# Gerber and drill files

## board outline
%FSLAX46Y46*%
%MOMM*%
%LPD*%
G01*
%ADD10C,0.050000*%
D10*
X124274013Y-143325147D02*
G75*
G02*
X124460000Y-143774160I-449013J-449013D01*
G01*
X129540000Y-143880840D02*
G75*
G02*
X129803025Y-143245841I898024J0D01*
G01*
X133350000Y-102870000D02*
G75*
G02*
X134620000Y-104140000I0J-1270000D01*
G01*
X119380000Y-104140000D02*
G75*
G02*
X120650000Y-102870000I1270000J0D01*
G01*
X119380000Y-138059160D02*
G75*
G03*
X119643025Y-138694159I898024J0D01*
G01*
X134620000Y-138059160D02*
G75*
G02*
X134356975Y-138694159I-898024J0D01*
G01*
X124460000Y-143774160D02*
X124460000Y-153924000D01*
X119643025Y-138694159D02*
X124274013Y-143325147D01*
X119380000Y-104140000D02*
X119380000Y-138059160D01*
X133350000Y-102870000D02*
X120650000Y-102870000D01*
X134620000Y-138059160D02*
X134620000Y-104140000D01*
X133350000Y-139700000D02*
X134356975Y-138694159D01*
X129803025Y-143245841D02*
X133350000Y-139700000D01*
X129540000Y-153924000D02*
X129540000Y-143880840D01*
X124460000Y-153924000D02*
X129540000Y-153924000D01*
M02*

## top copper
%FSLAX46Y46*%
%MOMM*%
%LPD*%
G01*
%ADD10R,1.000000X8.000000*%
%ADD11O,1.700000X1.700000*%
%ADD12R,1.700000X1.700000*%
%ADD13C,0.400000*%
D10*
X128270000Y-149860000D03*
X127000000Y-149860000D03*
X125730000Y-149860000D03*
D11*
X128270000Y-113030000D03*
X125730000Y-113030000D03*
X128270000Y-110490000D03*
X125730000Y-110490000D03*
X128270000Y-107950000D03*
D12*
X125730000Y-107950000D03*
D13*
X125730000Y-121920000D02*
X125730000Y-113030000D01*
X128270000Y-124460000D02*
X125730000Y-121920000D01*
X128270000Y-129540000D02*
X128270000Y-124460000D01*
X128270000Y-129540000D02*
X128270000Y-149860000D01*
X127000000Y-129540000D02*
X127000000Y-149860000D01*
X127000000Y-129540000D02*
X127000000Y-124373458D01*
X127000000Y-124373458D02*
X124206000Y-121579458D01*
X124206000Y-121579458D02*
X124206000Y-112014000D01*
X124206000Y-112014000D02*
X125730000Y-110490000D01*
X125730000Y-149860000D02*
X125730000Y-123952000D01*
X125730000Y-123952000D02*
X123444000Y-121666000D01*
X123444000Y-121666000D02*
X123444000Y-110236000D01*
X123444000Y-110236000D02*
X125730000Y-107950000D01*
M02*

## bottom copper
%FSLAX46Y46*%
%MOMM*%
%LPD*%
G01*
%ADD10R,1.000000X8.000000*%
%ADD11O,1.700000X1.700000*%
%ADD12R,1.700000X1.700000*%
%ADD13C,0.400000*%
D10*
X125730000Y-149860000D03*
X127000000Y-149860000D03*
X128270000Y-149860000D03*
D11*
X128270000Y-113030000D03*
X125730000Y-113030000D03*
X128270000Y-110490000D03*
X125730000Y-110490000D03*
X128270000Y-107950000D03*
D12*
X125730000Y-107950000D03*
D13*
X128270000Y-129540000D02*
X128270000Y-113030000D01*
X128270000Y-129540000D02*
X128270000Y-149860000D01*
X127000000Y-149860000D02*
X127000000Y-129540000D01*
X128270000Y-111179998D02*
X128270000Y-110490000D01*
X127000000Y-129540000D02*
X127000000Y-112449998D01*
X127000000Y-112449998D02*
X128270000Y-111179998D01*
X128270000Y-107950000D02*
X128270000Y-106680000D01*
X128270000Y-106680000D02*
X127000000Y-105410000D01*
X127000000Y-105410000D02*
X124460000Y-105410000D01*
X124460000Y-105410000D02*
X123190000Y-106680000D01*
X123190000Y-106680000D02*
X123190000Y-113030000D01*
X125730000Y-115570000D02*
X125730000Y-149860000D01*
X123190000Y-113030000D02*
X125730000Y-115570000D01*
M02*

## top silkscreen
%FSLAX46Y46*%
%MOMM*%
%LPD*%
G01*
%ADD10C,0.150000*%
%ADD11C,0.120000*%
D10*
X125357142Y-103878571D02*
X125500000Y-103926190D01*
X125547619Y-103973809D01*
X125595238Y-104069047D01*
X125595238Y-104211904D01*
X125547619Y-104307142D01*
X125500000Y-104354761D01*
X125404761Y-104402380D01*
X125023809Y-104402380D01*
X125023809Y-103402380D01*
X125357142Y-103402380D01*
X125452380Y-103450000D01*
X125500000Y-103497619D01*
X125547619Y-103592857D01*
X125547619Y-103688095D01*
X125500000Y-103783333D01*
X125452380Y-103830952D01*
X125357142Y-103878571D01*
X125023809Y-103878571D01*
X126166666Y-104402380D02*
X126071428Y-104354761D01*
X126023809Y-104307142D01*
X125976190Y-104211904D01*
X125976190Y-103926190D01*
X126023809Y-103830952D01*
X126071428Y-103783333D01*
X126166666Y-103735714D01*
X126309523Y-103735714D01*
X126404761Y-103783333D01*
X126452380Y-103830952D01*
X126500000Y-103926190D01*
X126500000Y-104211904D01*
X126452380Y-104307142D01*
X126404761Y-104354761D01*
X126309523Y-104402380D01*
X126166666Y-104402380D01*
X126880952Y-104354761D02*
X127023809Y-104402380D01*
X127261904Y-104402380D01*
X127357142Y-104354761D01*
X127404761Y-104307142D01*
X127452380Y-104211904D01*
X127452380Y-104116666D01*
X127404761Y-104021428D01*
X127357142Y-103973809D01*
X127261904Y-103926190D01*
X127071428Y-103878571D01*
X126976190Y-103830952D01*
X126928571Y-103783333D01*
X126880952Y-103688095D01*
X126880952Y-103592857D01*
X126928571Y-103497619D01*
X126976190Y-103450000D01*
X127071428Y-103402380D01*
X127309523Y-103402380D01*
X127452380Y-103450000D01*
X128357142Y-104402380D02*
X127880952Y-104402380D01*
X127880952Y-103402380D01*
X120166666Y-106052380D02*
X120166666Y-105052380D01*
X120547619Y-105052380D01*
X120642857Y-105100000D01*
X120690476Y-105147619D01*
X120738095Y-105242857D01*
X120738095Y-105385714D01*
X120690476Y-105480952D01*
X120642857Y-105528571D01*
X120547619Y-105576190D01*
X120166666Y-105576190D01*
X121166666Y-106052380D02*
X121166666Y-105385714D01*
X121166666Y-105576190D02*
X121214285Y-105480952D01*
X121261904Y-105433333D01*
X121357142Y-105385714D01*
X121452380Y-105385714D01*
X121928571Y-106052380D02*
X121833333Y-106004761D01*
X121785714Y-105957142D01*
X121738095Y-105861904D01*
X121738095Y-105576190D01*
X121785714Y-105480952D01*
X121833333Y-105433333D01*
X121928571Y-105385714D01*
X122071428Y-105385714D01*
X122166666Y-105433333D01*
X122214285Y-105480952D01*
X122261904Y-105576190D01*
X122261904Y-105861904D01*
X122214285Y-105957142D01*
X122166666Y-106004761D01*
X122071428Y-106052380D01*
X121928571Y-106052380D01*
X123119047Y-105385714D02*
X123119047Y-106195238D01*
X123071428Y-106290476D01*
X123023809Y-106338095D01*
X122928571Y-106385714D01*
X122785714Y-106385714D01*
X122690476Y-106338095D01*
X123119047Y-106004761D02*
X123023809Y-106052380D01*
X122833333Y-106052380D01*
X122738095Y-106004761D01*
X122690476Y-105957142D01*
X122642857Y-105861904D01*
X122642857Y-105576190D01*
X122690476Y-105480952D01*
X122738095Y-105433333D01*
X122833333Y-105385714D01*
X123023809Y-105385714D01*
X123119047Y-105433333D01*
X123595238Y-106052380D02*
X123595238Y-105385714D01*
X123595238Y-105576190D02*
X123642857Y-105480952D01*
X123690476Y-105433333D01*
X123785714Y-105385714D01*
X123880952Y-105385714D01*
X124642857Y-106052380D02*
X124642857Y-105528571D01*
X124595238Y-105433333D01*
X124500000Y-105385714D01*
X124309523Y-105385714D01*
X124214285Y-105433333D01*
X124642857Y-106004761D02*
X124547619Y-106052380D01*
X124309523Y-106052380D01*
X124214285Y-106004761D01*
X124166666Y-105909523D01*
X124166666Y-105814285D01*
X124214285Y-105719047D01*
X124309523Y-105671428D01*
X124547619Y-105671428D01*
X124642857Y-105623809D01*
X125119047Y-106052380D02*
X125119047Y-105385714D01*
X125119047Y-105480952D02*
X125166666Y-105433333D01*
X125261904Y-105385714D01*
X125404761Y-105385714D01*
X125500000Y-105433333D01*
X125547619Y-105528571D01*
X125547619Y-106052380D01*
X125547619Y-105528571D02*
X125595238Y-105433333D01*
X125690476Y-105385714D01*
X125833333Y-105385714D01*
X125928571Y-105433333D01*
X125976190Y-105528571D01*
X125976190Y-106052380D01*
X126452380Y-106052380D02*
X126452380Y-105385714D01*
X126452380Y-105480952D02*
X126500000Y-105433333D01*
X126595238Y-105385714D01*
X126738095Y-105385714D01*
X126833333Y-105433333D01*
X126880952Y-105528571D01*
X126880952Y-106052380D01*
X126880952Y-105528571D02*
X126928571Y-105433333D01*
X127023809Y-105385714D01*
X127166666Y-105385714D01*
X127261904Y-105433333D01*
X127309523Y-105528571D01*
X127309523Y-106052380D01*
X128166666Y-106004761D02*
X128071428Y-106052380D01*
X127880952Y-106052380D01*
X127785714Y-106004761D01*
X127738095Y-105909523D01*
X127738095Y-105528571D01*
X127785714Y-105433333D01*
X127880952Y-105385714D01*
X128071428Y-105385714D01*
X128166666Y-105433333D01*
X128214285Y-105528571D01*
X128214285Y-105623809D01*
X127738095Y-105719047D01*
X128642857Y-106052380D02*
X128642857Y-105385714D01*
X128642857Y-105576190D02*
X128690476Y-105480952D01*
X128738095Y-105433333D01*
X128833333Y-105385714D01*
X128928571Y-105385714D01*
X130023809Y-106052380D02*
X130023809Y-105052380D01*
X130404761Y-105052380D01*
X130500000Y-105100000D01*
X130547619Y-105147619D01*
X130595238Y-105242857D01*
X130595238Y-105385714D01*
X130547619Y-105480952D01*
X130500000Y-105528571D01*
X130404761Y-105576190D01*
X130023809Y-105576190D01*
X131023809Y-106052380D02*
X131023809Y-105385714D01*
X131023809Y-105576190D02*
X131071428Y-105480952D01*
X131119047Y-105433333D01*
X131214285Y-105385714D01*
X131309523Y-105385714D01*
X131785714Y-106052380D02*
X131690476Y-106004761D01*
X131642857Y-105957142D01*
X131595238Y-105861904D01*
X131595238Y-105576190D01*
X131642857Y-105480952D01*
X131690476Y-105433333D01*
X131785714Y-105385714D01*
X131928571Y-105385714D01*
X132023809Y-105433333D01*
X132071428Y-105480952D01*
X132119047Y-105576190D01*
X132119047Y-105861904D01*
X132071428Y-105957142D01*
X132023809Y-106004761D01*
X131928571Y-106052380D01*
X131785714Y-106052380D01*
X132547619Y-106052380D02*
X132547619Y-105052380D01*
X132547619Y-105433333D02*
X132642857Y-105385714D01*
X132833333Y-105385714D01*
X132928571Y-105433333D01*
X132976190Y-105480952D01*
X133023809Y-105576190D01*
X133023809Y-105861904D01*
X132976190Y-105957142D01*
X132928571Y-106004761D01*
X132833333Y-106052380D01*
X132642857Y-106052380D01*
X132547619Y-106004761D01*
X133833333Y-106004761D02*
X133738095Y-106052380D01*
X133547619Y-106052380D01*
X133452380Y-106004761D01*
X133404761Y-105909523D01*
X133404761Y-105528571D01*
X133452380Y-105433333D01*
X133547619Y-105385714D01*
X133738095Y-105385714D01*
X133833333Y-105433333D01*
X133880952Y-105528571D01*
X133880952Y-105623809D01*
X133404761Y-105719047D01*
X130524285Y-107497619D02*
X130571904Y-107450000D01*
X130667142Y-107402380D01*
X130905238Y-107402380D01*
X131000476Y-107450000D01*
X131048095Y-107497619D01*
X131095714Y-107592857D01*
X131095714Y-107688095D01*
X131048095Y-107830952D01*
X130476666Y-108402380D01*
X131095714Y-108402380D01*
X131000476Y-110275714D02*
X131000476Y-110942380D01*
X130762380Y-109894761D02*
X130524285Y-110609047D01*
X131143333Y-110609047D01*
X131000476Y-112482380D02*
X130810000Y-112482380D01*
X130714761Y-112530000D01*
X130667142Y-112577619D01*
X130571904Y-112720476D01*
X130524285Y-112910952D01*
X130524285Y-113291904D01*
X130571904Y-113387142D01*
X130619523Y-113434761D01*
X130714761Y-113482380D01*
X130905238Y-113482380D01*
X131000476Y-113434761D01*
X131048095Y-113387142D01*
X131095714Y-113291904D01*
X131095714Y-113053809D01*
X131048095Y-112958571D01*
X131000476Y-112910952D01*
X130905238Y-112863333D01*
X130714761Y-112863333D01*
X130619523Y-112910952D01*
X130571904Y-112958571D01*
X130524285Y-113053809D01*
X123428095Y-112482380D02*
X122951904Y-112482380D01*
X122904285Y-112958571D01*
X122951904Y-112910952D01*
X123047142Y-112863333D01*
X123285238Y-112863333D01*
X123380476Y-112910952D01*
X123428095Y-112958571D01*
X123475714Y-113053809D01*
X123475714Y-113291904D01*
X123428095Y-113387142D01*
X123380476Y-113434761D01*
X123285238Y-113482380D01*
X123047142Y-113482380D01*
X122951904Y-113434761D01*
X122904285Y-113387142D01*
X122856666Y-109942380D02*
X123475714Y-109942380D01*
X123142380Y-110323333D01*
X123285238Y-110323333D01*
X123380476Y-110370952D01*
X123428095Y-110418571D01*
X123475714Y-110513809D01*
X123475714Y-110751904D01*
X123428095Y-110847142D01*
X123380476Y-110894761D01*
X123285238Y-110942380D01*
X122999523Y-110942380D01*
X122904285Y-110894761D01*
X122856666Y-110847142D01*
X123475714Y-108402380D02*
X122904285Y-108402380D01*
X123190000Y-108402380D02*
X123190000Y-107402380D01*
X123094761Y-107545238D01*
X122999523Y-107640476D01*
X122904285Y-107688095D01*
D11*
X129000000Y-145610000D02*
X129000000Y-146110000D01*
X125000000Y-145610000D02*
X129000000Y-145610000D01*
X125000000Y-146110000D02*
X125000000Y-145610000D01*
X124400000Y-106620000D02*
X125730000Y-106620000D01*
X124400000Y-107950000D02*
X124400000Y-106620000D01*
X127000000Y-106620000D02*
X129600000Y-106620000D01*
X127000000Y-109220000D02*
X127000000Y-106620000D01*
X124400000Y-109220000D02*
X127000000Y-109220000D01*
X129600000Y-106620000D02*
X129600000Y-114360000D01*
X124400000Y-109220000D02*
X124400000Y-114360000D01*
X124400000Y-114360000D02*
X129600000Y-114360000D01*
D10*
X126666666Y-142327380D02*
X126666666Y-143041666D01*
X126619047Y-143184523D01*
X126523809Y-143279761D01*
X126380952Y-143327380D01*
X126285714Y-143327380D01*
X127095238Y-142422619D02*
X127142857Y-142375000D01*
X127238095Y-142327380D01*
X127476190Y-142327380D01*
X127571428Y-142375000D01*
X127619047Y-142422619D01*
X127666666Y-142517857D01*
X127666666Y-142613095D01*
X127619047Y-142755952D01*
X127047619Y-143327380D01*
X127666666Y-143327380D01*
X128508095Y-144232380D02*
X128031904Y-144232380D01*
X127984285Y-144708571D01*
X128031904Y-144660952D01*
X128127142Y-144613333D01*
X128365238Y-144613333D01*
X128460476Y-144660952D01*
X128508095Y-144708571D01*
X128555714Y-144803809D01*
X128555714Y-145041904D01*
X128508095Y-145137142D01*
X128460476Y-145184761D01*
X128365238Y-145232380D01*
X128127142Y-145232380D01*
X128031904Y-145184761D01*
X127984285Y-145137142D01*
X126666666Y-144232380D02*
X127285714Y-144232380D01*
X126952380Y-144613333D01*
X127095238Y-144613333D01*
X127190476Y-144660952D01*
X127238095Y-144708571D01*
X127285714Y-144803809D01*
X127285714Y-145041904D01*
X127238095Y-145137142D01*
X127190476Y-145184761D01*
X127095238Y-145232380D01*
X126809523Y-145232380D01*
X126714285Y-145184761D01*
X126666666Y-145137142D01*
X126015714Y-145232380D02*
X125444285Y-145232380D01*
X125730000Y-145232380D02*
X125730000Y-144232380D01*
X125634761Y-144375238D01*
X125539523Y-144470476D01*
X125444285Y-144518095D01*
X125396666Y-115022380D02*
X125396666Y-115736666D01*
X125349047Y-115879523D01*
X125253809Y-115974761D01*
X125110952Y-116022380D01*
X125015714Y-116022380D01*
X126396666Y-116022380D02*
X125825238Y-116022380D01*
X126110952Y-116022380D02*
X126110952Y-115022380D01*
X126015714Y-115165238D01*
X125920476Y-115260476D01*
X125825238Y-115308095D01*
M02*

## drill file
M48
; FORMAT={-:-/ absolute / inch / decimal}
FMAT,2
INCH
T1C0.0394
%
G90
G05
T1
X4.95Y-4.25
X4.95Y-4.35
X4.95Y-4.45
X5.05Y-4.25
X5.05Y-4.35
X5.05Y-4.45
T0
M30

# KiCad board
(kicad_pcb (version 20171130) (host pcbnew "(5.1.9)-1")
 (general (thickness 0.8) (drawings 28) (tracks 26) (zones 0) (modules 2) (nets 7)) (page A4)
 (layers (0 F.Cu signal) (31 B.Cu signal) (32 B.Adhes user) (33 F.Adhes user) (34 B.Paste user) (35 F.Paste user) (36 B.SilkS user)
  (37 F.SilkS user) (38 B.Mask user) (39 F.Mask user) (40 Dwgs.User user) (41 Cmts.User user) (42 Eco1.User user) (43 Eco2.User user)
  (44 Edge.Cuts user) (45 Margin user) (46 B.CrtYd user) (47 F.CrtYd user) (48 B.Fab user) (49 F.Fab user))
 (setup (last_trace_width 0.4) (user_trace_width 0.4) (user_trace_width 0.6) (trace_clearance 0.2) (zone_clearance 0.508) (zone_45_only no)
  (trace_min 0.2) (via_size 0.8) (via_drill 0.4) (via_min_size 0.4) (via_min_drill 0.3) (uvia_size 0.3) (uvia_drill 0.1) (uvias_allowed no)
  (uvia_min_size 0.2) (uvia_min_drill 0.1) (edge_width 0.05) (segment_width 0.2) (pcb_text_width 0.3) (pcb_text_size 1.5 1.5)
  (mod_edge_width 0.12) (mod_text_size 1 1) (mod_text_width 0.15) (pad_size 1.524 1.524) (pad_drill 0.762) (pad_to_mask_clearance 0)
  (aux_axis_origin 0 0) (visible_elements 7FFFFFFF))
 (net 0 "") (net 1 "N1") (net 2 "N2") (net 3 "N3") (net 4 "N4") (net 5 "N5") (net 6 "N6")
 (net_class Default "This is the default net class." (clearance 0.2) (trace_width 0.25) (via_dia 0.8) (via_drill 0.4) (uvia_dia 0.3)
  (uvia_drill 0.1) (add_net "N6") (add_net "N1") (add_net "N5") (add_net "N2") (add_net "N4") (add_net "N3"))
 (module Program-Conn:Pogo (layer F.Cu) (at 127 149.86)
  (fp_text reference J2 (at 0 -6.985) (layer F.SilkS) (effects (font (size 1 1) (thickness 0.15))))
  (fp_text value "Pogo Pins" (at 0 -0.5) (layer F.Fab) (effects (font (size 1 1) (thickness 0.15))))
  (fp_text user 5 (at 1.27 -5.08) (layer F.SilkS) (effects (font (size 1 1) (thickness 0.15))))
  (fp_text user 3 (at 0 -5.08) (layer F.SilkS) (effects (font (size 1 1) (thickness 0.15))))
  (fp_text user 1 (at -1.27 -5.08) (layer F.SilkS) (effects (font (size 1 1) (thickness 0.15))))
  (fp_line (start 2 -4.25) (end 2 -3.75) (layer F.SilkS) (width 0.12))
  (fp_line (start -2 -4.25) (end 2 -4.25) (layer F.SilkS) (width 0.12))
  (fp_line (start -2 -3.75) (end -2 -4.25) (layer F.SilkS) (width 0.12))
  (pad 2 smd rect (at -1.27 0) (size 1 8) (layers B.Cu B.Paste B.Mask) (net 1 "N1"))
  (pad 4 smd rect (at 0 0) (size 1 8) (layers B.Cu B.Paste B.Mask) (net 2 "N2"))
  (pad 6 smd rect (at 1.27 0) (size 1 8) (layers B.Cu B.Paste B.Mask) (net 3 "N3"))
  (pad 5 smd rect (at 1.27 0) (size 1 8) (layers F.Cu F.Paste F.Mask) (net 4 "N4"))
  (pad 3 smd rect (at 0 0) (size 1 8) (layers F.Cu F.Paste F.Mask) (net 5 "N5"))
  (pad 1 smd rect (at -1.27 0) (size 1 8) (layers F.Cu F.Paste F.Mask) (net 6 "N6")))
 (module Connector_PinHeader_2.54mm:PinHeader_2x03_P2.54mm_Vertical (layer F.Cu) (at 125.73 107.95)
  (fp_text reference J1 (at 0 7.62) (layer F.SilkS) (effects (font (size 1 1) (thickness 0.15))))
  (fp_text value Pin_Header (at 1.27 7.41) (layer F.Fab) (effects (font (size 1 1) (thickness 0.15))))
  (fp_line (start -1.33 -1.33) (end 0 -1.33) (layer F.SilkS) (width 0.12))
  (fp_line (start -1.33 0) (end -1.33 -1.33) (layer F.SilkS) (width 0.12))
  (fp_line (start 1.27 -1.33) (end 3.87 -1.33) (layer F.SilkS) (width 0.12))
  (fp_line (start 1.27 1.27) (end 1.27 -1.33) (layer F.SilkS) (width 0.12))
  (fp_line (start -1.33 1.27) (end 1.27 1.27) (layer F.SilkS) (width 0.12))
  (fp_line (start 3.87 -1.33) (end 3.87 6.41) (layer F.SilkS) (width 0.12))
  (fp_line (start -1.33 1.27) (end -1.33 6.41) (layer F.SilkS) (width 0.12))
  (fp_line (start -1.33 6.41) (end 3.87 6.41) (layer F.SilkS) (width 0.12))
  (pad 6 thru_hole oval (at 2.54 5.08) (size 1.7 1.7) (drill 1) (layers *.Cu *.Mask) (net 3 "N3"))
  (pad 5 thru_hole oval (at 0 5.08) (size 1.7 1.7) (drill 1) (layers *.Cu *.Mask) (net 4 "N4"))
  (pad 4 thru_hole oval (at 2.54 2.54) (size 1.7 1.7) (drill 1) (layers *.Cu *.Mask) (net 2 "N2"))
  (pad 3 thru_hole oval (at 0 2.54) (size 1.7 1.7) (drill 1) (layers *.Cu *.Mask) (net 5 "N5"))
  (pad 2 thru_hole oval (at 2.54 0) (size 1.7 1.7) (drill 1) (layers *.Cu *.Mask) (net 1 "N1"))
  (pad 1 thru_hole rect (at 0 0) (size 1.7 1.7) (drill 1) (layers *.Cu *.Mask) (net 6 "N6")))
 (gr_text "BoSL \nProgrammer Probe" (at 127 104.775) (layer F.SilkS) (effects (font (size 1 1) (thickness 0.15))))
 (gr_arc (start 123.825 143.77416) (end 124.46 143.77416) (angle -45) (layer Edge.Cuts) (width 0.05))
 (gr_arc (start 130.438024 143.88084) (end 129.803025 143.245841) (angle -45) (layer Edge.Cuts) (width 0.05))
 (gr_arc (start 133.35 104.14) (end 134.62 104.14) (angle -90) (layer Edge.Cuts) (width 0.05))
 (gr_arc (start 120.65 104.14) (end 120.65 102.87) (angle -90) (layer Edge.Cuts) (width 0.05))
 (gr_arc (start 120.278024 138.05916) (end 119.643025 138.694159) (angle 45) (layer Edge.Cuts) (width 0.05))
 (gr_arc (start 133.721976 138.05916) (end 134.356975 138.694159) (angle -45) (layer Edge.Cuts) (width 0.05))
 (gr_line (start 124.46 143.77416) (end 124.46 153.924) (layer Edge.Cuts) (width 0.05))
 (gr_line (start 119.643025 138.694159) (end 124.274013 143.325147) (layer Edge.Cuts) (width 0.05))
 (gr_line (start 119.38 104.14) (end 119.38 138.05916) (layer Edge.Cuts) (width 0.05))
 (gr_line (start 133.35 102.87) (end 120.65 102.87) (layer Edge.Cuts) (width 0.05))
 (gr_line (start 134.62 138.05916) (end 134.62 104.14) (layer Edge.Cuts) (width 0.05))
 (gr_line (start 133.35 139.7) (end 134.356975 138.694159) (layer Edge.Cuts) (width 0.05))
 (gr_line (start 129.803025 143.245841) (end 133.35 139.7) (layer Edge.Cuts) (width 0.05))
 (gr_line (start 129.54 153.924) (end 129.54 143.88084) (layer Edge.Cuts) (width 0.05))
 (gr_line (start 124.46 153.924) (end 129.54 153.924) (layer Edge.Cuts) (width 0.05))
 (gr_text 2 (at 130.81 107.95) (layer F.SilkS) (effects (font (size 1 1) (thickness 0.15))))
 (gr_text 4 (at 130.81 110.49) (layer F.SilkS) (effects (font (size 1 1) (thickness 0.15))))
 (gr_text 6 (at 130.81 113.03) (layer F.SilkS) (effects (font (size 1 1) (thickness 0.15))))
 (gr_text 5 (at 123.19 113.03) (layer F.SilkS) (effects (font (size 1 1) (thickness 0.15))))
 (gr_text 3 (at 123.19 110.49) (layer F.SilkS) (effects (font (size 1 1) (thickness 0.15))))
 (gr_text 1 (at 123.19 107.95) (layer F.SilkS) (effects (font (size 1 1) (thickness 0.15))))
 (segment (start 128.27 129.54) (end 128.27 113.03) (width 0.4) (layer B.Cu) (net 3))
 (segment (start 128.27 129.54) (end 128.27 149.86) (width 0.4) (layer B.Cu) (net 3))
 (segment (start 125.73 121.92) (end 125.73 113.03) (width 0.4) (layer F.Cu) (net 4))
 (segment (start 128.27 124.46) (end 125.73 121.92) (width 0.4) (layer F.Cu) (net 4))
 (segment (start 128.27 129.54) (end 128.27 124.46) (width 0.4) (layer F.Cu) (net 4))
 (segment (start 128.27 129.54) (end 128.27 149.86) (width 0.4) (layer F.Cu) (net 4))
 (segment (start 127 149.86) (end 127 129.54) (width 0.4) (layer B.Cu) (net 2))
 (segment (start 128.27 111.179998) (end 128.27 110.49) (width 0.4) (layer B.Cu) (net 2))
 (segment (start 127 129.54) (end 127 112.449998) (width 0.4) (layer B.Cu) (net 2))
 (segment (start 127 112.449998) (end 128.27 111.179998) (width 0.4) (layer B.Cu) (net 2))
 (segment (start 127 129.54) (end 127 149.86) (width 0.4) (layer F.Cu) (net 5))
 (segment (start 127 129.54) (end 127 124.373458) (width 0.4) (layer F.Cu) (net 5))
 (segment (start 127 124.373458) (end 124.206 121.579458) (width 0.4) (layer F.Cu) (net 5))
 (segment (start 124.206 121.579458) (end 124.206 112.014) (width 0.4) (layer F.Cu) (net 5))
 (segment (start 124.206 112.014) (end 125.73 110.49) (width 0.4) (layer F.Cu) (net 5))
 (segment (start 128.27 107.95) (end 128.27 106.68) (width 0.4) (layer B.Cu) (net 1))
 (segment (start 128.27 106.68) (end 127 105.41) (width 0.4) (layer B.Cu) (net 1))
 (segment (start 127 105.41) (end 124.46 105.41) (width 0.4) (layer B.Cu) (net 1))
 (segment (start 124.46 105.41) (end 123.19 106.68) (width 0.4) (layer B.Cu) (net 1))
 (segment (start 123.19 106.68) (end 123.19 113.03) (width 0.4) (layer B.Cu) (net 1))
 (segment (start 125.73 115.57) (end 125.73 149.86) (width 0.4) (layer B.Cu) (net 1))
 (segment (start 123.19 113.03) (end 125.73 115.57) (width 0.4) (layer B.Cu) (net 1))
 (segment (start 125.73 149.86) (end 125.73 123.952) (width 0.4) (layer F.Cu) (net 6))
 (segment (start 125.73 123.952) (end 123.444 121.666) (width 0.4) (layer F.Cu) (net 6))
 (segment (start 123.444 121.666) (end 123.444 110.236) (width 0.4) (layer F.Cu) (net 6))
 (segment (start 123.444 110.236) (end 125.73 107.95) (width 0.4) (layer F.Cu) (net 6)))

